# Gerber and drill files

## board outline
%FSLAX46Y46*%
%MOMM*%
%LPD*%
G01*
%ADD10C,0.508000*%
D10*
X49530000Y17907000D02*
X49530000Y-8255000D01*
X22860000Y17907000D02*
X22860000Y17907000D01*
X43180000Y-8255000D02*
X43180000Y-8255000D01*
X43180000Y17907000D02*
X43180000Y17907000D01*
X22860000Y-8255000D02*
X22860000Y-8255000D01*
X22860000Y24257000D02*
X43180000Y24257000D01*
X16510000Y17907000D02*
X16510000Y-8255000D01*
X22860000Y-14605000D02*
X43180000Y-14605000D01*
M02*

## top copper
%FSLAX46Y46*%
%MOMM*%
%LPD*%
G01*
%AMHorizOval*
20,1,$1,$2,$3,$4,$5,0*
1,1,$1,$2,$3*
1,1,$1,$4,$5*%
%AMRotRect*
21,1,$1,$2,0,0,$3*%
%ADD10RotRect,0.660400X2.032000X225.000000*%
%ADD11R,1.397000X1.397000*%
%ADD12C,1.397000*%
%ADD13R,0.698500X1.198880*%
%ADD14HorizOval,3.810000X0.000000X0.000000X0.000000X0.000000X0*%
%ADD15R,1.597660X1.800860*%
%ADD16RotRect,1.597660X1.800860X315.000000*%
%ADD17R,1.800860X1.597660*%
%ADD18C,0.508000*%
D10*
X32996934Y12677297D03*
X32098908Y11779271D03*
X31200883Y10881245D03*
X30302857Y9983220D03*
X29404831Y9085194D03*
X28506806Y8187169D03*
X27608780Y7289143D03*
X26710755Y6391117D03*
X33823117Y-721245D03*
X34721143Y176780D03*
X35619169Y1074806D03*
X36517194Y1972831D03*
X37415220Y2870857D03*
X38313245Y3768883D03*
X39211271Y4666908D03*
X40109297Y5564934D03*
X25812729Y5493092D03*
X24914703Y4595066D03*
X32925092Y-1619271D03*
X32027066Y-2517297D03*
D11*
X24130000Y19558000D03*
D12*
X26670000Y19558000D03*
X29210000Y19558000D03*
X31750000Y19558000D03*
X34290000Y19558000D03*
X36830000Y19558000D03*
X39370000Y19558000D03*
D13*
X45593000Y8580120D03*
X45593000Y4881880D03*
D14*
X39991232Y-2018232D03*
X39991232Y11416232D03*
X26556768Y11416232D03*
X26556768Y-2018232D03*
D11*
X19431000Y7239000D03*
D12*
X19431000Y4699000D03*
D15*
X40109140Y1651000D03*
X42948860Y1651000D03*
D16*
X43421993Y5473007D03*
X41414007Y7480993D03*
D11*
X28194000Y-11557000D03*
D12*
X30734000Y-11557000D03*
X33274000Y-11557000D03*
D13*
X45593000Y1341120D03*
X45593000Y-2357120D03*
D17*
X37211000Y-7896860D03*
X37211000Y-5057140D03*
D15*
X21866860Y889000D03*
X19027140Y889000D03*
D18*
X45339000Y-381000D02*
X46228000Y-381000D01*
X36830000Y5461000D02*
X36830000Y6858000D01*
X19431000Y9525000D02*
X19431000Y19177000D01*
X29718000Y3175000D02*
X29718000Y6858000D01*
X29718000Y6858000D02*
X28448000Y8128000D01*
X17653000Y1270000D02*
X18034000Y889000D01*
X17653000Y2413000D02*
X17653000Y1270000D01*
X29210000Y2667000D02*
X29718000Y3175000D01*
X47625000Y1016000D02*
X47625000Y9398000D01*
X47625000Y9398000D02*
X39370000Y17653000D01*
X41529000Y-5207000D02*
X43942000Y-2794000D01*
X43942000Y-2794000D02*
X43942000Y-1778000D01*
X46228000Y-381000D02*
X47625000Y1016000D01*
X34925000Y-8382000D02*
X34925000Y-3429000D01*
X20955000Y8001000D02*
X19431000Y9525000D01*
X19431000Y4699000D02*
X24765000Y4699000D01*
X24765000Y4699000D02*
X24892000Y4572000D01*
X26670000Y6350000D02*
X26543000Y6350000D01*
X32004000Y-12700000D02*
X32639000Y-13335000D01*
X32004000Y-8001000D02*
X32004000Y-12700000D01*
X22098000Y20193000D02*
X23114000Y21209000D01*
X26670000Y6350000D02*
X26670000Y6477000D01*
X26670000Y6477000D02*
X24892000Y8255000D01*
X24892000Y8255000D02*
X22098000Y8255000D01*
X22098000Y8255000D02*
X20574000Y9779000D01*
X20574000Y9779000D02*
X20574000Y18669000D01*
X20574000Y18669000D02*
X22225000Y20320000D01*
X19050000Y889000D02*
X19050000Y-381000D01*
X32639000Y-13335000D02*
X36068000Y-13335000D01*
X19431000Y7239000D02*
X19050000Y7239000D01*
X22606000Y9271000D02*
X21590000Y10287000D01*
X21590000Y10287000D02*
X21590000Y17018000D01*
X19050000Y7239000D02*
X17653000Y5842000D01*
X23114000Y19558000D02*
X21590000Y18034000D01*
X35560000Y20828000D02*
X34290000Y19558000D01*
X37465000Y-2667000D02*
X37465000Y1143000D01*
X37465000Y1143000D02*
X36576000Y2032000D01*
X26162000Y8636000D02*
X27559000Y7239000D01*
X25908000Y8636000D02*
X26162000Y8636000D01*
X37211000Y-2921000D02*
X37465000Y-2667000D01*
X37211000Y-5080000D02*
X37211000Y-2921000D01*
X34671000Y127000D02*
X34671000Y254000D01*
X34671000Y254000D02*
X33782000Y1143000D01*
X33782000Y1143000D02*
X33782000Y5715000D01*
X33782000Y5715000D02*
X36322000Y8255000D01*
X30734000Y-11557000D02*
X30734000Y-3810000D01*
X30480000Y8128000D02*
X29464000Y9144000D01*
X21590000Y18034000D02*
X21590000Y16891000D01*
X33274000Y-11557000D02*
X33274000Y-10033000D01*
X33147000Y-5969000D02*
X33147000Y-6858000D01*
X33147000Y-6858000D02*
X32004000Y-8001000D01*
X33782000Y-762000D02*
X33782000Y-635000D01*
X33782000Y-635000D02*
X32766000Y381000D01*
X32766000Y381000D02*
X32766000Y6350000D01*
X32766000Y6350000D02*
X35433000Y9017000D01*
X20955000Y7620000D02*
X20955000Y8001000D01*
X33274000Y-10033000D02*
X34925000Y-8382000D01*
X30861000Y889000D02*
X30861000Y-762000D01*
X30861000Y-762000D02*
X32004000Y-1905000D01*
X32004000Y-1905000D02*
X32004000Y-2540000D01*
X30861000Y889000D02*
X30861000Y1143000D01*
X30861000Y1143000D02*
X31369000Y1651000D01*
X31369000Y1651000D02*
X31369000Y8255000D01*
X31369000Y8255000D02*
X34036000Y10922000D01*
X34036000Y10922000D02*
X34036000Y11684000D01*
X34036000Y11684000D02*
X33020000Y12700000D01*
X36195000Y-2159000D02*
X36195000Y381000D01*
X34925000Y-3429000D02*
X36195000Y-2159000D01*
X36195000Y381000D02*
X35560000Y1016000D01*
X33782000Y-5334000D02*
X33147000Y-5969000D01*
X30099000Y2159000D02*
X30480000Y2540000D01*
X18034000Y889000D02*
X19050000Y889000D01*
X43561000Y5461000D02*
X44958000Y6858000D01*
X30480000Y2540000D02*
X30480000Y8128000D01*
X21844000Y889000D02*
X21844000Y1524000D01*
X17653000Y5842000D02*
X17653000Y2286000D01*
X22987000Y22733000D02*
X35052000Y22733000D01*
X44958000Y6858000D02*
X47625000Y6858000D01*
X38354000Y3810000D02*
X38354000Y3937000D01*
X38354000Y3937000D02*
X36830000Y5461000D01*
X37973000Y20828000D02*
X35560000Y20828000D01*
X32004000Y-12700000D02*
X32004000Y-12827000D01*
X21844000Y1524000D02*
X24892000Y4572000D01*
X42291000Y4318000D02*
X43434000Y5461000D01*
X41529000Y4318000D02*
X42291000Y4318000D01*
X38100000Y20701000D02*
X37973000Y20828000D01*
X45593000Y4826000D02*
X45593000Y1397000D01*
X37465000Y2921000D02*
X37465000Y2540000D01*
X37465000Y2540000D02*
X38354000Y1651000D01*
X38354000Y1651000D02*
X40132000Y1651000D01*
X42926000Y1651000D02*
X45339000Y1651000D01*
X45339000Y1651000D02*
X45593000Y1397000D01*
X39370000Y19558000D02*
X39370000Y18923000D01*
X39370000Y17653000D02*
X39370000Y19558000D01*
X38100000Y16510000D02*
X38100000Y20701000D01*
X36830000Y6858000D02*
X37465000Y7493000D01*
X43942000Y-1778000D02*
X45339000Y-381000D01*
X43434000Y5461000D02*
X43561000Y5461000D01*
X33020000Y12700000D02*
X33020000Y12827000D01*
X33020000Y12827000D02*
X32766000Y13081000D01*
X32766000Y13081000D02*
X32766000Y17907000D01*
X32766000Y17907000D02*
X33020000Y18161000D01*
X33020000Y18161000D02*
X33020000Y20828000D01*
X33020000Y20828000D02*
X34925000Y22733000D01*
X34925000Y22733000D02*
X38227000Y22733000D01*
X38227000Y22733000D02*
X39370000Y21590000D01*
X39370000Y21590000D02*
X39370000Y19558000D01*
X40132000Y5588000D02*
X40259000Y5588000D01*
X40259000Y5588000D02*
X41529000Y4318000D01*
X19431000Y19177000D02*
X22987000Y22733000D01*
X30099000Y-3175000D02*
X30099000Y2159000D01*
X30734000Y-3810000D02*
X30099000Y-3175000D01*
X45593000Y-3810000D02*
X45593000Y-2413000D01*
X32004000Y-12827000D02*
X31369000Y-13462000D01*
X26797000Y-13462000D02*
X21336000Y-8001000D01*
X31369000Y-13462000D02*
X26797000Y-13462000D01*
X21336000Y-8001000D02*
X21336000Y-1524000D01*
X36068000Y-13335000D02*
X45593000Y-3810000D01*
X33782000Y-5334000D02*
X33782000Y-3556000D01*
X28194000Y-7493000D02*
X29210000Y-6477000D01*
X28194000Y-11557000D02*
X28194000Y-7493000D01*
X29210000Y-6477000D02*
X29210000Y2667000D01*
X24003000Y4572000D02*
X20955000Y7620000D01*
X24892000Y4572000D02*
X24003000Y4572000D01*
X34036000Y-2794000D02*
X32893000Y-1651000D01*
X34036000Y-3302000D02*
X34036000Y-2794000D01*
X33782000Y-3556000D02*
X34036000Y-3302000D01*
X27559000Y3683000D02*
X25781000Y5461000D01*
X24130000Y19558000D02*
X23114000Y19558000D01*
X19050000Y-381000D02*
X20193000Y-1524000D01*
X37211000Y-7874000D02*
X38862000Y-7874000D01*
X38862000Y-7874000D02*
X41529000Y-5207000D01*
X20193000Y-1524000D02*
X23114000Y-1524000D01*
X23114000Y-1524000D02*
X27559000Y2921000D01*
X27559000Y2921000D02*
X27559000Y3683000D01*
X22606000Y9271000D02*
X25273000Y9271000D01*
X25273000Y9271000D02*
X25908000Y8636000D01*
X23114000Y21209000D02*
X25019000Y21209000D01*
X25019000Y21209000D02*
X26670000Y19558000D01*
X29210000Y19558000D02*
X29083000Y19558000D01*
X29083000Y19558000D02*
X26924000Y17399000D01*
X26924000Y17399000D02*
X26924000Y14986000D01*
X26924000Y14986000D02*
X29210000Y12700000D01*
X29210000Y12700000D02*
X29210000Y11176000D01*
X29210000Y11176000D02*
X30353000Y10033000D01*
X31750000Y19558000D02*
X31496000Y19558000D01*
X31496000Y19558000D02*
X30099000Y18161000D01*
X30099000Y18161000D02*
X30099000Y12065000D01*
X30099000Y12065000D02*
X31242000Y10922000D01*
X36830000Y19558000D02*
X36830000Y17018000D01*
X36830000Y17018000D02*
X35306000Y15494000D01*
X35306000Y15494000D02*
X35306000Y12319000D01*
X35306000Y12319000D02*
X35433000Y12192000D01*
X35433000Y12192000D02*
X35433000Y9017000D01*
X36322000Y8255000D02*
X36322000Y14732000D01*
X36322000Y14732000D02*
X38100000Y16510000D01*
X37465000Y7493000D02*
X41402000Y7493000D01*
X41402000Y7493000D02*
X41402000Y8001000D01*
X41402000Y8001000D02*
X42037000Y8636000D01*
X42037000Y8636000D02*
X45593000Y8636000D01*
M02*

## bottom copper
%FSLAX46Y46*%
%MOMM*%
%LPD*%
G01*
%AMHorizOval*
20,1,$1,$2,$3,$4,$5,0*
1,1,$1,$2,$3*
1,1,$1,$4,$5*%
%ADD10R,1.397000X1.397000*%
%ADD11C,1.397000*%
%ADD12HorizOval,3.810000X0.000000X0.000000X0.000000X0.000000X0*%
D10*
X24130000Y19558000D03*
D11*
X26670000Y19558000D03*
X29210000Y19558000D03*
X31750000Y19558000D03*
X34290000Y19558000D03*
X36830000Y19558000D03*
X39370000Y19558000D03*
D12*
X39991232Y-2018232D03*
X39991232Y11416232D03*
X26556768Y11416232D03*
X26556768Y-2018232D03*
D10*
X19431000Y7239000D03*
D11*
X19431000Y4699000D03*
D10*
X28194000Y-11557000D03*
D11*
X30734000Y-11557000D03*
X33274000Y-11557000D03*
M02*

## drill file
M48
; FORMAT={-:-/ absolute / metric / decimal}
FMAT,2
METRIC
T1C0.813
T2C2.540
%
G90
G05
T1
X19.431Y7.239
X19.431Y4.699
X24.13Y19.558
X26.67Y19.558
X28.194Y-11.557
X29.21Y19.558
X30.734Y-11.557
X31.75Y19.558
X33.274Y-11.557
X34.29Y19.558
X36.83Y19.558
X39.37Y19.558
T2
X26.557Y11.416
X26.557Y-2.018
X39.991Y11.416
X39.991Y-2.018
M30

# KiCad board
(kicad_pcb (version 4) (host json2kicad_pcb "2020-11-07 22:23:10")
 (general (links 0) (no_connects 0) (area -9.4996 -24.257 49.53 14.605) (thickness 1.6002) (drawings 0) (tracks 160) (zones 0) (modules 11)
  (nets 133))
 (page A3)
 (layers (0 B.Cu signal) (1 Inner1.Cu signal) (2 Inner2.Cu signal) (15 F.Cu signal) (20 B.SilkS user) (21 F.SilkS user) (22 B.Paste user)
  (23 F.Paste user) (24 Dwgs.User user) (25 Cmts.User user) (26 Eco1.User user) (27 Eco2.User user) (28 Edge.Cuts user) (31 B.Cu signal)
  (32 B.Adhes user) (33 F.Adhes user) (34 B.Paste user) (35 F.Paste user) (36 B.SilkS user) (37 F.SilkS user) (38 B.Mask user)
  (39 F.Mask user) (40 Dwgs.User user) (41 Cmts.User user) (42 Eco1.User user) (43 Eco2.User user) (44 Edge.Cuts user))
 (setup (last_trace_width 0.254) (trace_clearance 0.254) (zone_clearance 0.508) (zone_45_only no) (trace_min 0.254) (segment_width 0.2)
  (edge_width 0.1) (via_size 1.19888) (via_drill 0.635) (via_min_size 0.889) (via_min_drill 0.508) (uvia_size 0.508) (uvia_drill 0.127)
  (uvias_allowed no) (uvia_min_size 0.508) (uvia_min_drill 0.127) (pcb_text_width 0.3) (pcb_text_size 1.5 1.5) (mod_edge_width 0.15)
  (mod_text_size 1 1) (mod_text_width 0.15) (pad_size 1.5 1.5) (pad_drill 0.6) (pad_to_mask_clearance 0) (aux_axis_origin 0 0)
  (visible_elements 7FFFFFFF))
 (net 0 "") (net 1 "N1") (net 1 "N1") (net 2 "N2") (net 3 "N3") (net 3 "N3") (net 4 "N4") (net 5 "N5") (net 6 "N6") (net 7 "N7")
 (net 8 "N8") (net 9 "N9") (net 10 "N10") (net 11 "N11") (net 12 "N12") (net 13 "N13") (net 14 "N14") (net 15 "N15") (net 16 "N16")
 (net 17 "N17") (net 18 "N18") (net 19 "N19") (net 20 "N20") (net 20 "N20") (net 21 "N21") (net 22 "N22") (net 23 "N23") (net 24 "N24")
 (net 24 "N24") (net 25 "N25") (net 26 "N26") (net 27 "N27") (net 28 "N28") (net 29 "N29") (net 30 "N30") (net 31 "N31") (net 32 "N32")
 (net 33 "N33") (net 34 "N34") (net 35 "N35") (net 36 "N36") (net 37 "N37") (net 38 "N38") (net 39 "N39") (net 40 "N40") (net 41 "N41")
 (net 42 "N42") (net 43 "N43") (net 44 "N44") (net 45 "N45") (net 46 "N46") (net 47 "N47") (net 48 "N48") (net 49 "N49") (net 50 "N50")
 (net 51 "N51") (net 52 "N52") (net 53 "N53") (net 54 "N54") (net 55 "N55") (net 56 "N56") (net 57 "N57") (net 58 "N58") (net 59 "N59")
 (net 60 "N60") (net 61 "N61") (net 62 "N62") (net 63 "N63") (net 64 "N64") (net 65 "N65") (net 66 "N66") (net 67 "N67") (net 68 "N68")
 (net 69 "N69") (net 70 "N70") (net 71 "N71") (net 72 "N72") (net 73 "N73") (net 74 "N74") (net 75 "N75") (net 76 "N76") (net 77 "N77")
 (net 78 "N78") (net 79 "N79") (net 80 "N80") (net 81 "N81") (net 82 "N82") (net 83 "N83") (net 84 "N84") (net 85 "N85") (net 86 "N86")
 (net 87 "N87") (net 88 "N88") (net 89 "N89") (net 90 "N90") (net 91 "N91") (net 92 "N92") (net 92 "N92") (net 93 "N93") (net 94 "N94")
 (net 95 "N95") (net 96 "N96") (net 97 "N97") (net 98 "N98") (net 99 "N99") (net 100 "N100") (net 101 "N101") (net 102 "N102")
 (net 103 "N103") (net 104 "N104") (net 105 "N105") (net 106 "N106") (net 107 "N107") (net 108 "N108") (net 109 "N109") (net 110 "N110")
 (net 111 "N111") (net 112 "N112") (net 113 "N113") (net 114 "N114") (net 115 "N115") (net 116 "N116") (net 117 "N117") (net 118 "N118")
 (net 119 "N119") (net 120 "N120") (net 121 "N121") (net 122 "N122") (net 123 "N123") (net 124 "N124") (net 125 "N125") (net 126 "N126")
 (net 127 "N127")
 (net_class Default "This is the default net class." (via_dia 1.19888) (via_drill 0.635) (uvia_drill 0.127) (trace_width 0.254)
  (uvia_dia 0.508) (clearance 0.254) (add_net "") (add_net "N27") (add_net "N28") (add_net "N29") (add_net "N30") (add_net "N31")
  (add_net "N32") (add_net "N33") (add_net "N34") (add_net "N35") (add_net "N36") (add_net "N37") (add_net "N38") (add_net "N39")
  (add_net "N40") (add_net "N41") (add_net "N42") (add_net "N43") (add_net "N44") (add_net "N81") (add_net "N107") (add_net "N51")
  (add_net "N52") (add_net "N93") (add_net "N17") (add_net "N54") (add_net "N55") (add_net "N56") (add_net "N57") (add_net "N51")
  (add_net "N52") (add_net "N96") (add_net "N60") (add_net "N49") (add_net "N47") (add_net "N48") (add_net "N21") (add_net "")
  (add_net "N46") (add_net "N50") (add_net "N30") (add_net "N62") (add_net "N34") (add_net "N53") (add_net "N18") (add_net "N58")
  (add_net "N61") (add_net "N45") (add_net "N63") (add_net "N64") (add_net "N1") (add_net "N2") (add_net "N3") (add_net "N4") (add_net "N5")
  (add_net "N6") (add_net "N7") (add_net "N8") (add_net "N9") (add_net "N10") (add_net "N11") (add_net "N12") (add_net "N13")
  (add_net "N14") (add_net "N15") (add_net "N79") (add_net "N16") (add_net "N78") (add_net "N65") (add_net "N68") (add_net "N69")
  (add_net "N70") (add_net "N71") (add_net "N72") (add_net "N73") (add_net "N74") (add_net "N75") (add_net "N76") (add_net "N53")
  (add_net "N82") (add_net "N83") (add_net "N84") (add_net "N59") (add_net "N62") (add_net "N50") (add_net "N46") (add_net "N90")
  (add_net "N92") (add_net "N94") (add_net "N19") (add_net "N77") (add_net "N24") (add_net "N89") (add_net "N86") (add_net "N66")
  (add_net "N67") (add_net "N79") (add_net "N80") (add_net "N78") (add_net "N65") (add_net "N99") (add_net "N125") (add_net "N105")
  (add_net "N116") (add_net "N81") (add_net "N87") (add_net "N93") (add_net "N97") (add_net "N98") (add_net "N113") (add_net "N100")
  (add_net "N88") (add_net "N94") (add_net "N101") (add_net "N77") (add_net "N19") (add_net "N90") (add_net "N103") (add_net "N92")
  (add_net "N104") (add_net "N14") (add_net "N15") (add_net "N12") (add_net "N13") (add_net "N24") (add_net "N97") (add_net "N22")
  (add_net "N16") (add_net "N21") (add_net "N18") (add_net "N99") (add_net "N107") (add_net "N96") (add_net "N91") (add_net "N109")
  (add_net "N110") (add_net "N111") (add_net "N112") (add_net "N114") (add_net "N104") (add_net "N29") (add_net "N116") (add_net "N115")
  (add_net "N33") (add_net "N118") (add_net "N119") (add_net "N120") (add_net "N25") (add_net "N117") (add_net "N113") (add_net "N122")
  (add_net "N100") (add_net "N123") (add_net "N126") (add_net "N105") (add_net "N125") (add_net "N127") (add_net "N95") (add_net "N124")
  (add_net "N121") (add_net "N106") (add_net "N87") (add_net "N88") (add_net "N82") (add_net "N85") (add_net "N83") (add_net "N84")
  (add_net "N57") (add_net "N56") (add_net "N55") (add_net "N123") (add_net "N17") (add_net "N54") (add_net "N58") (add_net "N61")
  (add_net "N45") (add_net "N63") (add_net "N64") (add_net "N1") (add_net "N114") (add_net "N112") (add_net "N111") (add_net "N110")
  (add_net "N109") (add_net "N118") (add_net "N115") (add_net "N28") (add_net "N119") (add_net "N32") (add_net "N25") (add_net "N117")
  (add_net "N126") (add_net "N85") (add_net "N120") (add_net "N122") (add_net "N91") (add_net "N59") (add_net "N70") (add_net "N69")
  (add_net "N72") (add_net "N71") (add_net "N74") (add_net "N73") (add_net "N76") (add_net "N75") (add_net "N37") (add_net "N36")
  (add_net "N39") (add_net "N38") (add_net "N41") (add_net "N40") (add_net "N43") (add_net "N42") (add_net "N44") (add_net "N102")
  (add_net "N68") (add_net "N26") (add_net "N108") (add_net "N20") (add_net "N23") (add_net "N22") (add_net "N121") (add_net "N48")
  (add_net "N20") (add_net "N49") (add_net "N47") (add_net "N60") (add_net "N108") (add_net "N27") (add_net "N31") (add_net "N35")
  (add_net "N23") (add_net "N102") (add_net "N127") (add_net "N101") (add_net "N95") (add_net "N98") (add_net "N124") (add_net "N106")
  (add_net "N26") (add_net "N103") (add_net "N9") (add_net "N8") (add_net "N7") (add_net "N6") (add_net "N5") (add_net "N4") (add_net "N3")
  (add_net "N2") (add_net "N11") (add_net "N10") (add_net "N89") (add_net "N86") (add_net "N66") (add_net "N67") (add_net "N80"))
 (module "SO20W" (layer "F.Cu") (at 32.512 -5.08 -135.00)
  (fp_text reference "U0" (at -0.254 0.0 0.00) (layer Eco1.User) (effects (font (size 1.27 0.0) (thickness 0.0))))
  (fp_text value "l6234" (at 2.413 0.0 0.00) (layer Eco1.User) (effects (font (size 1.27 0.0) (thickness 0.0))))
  (pad 1 smd rect (at -5.715 5.0292 -135.00) (size 0.6604 2.032) (drill 0.0) (layers "F.Cu" "F.Paste") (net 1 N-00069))
  (pad 2 smd rect (at -4.445 5.0292 -135.00) (size 0.6604 2.032) (drill 0.0) (layers "F.Cu" "F.Paste") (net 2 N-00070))
  (pad 3 smd rect (at -3.175 5.0292 -135.00) (size 0.6604 2.032) (drill 0.0) (layers "F.Cu" "F.Paste") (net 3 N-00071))
  (pad 4 smd rect (at -1.905 5.0292 -135.00) (size 0.6604 2.032) (drill 0.0) (layers "F.Cu" "F.Paste") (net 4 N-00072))
  (pad 5 smd rect (at -0.635 5.0292 -135.00) (size 0.6604 2.032) (drill 0.0) (layers "F.Cu" "F.Paste") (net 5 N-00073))
  (pad 6 smd rect (at 0.635 5.0292 -135.00) (size 0.6604 2.032) (drill 0.0) (layers "F.Cu" "F.Paste") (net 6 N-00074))
  (pad 7 smd rect (at 1.905 5.0292 -135.00) (size 0.6604 2.032) (drill 0.0) (layers "F.Cu" "F.Paste") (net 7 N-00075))
  (pad 8 smd rect (at 3.175 5.0292 -135.00) (size 0.6604 2.032) (drill 0.0) (layers "F.Cu" "F.Paste") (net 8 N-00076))
  (pad 13 smd rect (at 3.175 -5.0292 -135.00) (size 0.6604 2.032) (drill 0.0) (layers "F.Cu" "F.Paste") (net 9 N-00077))
  (pad 14 smd rect (at 1.905 -5.0292 -135.00) (size 0.6604 2.032) (drill 0.0) (layers "F.Cu" "F.Paste") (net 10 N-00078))
  (pad 15 smd rect (at 0.635 -5.0292 -135.00) (size 0.6604 2.032) (drill 0.0) (layers "F.Cu" "F.Paste") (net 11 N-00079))
  (pad 16 smd rect (at -0.635 -5.0292 -135.00) (size 0.6604 2.032) (drill 0.0) (layers "F.Cu" "F.Paste") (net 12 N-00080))
  (pad 17 smd rect (at -1.905 -5.0292 -135.00) (size 0.6604 2.032) (drill 0.0) (layers "F.Cu" "F.Paste") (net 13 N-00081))
  (pad 18 smd rect (at -3.175 -5.0292 -135.00) (size 0.6604 2.032) (drill 0.0) (layers "F.Cu" "F.Paste") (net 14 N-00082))
  (pad 19 smd rect (at -4.445 -5.0292 -135.00) (size 0.6604 2.032) (drill 0.0) (layers "F.Cu" "F.Paste") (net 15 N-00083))
  (pad 20 smd rect (at -5.715 -5.0292 -135.00) (size 0.6604 2.032) (drill 0.0) (layers "F.Cu" "F.Paste") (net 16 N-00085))
  (pad 9 smd rect (at 4.445 5.0292 -135.00) (size 0.6604 2.032) (drill 0.0) (layers "F.Cu" "F.Paste") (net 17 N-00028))
  (pad 10 smd rect (at 5.715 5.0292 -135.00) (size 0.6604 2.032) (drill 0.0) (layers "F.Cu" "F.Paste") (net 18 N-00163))
  (pad 12 smd rect (at 4.445 -5.0292 -135.00) (size 0.6604 2.032) (drill 0.0) (layers "F.Cu" "F.Paste") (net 17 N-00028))
  (pad 11 smd rect (at 5.715 -5.0292 -135.00) (size 0.6604 2.032) (drill 0.0) (layers "F.Cu" "F.Paste") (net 1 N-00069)))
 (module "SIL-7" (layer "F.Cu") (at 31.75 -19.558 0.00)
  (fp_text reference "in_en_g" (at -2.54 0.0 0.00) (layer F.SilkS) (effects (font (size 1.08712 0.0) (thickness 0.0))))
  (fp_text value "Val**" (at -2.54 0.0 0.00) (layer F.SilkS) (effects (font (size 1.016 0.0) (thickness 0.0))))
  (pad 1 thru_hole rect (at -7.62 0.0 0.00) (size 1.397 1.397) (drill 0.8128)
   (layers "B.Cu" "Inner1.Cu" "Inner2.Cu" "F.Cu" "F.SilkS" "B.Paste" "F.Paste") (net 7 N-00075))
  (pad 2 thru_hole circle (at -5.08 0.0 0.00) (size 1.397 1.397) (drill 0.8128)
   (layers "B.Cu" "Inner1.Cu" "Inner2.Cu" "F.Cu" "B.SilkS" "F.SilkS" "B.Paste" "F.Paste") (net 8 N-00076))
  (pad 3 thru_hole circle (at -2.54 0.0 0.00) (size 1.397 1.397) (drill 0.8128)
   (layers "B.Cu" "Inner1.Cu" "Inner2.Cu" "F.Cu" "B.SilkS" "F.SilkS" "B.Paste" "F.Paste") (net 4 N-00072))
  (pad 4 thru_hole circle (at 0.0 0.0 0.00) (size 1.397 1.397) (drill 0.8128)
   (layers "B.Cu" "Inner1.Cu" "Inner2.Cu" "F.Cu" "B.SilkS" "F.SilkS" "B.Paste" "F.Paste") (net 3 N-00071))
  (pad 5 thru_hole circle (at 2.54 0.0 0.00) (size 1.397 1.397) (drill 0.8128)
   (layers "B.Cu" "Inner1.Cu" "Inner2.Cu" "F.Cu" "B.SilkS" "F.SilkS" "B.Paste" "F.Paste") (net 10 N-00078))
  (pad 6 thru_hole circle (at 5.08 0.0 0.00) (size 1.397 1.397) (drill 0.8128)
   (layers "B.Cu" "Inner1.Cu" "Inner2.Cu" "F.Cu" "B.SilkS" "F.SilkS" "B.Paste" "F.Paste") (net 9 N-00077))
  (pad 7 thru_hole circle (at 7.62 0.0 0.00) (size 1.397 1.397) (drill 0.8128)
   (layers "B.Cu" "Inner1.Cu" "Inner2.Cu" "F.Cu" "B.SilkS" "F.SilkS" "B.Paste" "F.Paste") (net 1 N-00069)))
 (segment (start 45.339 0.381) (end 46.228 0.381) (width 0.508) (layer F.Cu) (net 1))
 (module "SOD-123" (layer "F.Cu") (at 45.593 -6.731 -90.00)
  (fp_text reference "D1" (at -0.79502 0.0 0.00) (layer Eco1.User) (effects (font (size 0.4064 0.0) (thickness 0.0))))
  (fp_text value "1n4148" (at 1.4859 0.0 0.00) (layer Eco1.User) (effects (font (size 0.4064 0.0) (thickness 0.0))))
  (pad C smd rect (at -1.84912 0.0 -90.00) (size 1.19888 0.6985) (drill 0.0) (layers "F.Cu" "F.Paste") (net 14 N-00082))
  (pad A smd rect (at 1.84912 0.0 -90.00) (size 1.19888 0.6985) (drill 0.0) (layers "F.Cu" "F.Paste") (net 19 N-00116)))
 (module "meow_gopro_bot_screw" (layer "F.Cu") (at 33.274 -4.699 45.00)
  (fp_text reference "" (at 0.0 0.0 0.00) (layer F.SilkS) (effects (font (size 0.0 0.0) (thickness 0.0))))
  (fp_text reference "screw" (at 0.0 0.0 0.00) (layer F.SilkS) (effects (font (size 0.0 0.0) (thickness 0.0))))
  (pad S0 thru_hole oval (at 0.0 9.4996 45.00) (size 3.81 3.81) (drill 2.54)
   (layers "B.Cu" "Inner1.Cu" "Inner2.Cu" "F.Cu" "B.Paste" "F.Paste") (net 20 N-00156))
  (pad S1 thru_hole oval (at 9.4996 0.0 45.00) (size 3.81 3.81) (drill 2.54)
   (layers "B.Cu" "Inner1.Cu" "Inner2.Cu" "F.Cu" "B.Paste" "F.Paste") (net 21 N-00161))
  (pad S2 thru_hole oval (at 0.0 -9.4996 45.00) (size 3.81 3.81) (drill 2.54)
   (layers "B.Cu" "Inner1.Cu" "Inner2.Cu" "F.Cu" "B.Paste" "F.Paste") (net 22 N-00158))
  (pad S3 thru_hole oval (at -9.4996 0.0 45.00) (size 3.81 3.81) (drill 2.54)
   (layers "B.Cu" "Inner1.Cu" "Inner2.Cu" "F.Cu" "B.Paste" "F.Paste") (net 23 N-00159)))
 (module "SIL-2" (layer "F.Cu") (at 19.431 -5.969 -90.00)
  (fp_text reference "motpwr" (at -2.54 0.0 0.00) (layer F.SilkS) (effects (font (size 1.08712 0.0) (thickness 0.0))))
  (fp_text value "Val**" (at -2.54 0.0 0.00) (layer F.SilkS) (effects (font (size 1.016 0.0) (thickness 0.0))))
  (pad 1 thru_hole rect (at -1.27 0.0 -90.00) (size 1.397 1.397) (drill 0.8128)
   (layers "B.Cu" "Inner1.Cu" "Inner2.Cu" "F.Cu" "F.SilkS" "B.Paste" "F.Paste") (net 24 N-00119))
  (pad 2 thru_hole circle (at 1.27 0.0 -90.00) (size 1.397 1.397) (drill 0.8128)
   (layers "B.Cu" "Inner1.Cu" "Inner2.Cu" "F.Cu" "F.SilkS" "B.Paste" "F.Paste") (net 18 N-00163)))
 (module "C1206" (layer "F.Cu") (at 41.529 -1.651 180.00)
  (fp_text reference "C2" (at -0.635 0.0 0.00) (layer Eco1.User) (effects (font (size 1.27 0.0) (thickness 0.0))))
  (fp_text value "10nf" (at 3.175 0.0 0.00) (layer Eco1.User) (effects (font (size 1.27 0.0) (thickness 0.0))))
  (pad 2 smd rect (at 1.41986 0.0 -180.00) (size 1.59766 1.80086) (drill 0.0) (layers "F.Cu" "F.Paste") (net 13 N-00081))
  (pad 1 smd rect (at -1.41986 0.0 -180.00) (size 1.59766 1.80086) (drill 0.0) (layers "F.Cu" "F.Paste") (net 19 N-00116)))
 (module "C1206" (layer "F.Cu") (at 42.418 -6.477 -45.00)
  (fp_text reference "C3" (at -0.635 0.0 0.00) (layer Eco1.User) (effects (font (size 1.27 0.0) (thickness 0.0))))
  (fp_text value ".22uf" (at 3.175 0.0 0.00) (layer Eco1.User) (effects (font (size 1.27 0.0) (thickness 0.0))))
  (pad 2 smd rect (at 1.41986 0.0 -45.00) (size 1.59766 1.80086) (drill 0.0) (layers "F.Cu" "F.Paste") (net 16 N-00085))
  (pad 1 smd rect (at -1.41986 0.0 -45.00) (size 1.59766 1.80086) (drill 0.0) (layers "F.Cu" "F.Paste") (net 14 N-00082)))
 (segment (start 36.83 -5.461) (end 36.83 -6.858) (width 0.508) (layer F.Cu) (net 14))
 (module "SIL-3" (layer "F.Cu") (at 30.734 11.557 0.00)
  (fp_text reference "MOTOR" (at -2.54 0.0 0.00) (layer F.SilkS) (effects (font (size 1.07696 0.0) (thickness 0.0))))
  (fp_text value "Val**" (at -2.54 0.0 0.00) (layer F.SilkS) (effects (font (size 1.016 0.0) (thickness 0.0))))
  (pad 1 thru_hole rect (at -2.54 0.0 0.00) (size 1.397 1.397) (drill 0.8128)
   (layers "B.Cu" "Inner1.Cu" "Inner2.Cu" "F.Cu" "F.SilkS" "B.Paste" "F.Paste") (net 6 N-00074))
  (pad 2 thru_hole circle (at 0.0 0.0 0.00) (size 1.397 1.397) (drill 0.8128)
   (layers "B.Cu" "Inner1.Cu" "Inner2.Cu" "F.Cu" "F.SilkS" "B.Paste" "F.Paste") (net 5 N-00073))
  (pad 3 thru_hole circle (at 2.54 0.0 0.00) (size 1.397 1.397) (drill 0.8128)
   (layers "B.Cu" "Inner1.Cu" "Inner2.Cu" "F.Cu" "F.SilkS" "B.Paste" "F.Paste") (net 11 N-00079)))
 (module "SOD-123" (layer "F.Cu") (at 45.593 0.508 -90.00)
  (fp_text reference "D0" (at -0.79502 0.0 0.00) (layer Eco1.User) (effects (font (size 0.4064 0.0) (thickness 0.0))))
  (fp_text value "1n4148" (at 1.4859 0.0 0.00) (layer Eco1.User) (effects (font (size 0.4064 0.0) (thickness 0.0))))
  (pad C smd rect (at -1.84912 0.0 -90.00) (size 1.19888 0.6985) (drill 0.0) (layers "F.Cu" "F.Paste") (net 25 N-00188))
  (pad A smd rect (at 1.84912 0.0 -90.00) (size 1.19888 0.6985) (drill 0.0) (layers "F.Cu" "F.Paste") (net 17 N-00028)))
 (gr_line (start 49.53 -17.907) (end 49.53 8.255) (angle 51566.20) (width 0.508) (layer Edge.Cuts))
 (gr_line (start 22.86 -17.907) (end 22.86 -17.907) (angle -90.00) (width 0.508) (layer Edge.Cuts))
 (gr_line (start 43.18 8.255) (end 43.18 8.255) (angle -90.00) (width 0.508) (layer Edge.Cuts))
 (gr_line (start 43.18 -17.907) (end 43.18 -17.907) (angle -90.00) (width 0.508) (layer Edge.Cuts))
 (gr_line (start 22.86 8.255) (end 22.86 8.255) (angle -90.00) (width 0.508) (layer Edge.Cuts))
 (segment (start 19.431 -9.525) (end 19.431 -19.177) (width 0.508) (layer F.Cu) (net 1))
 (segment (start 29.718 -3.175) (end 29.718 -6.858) (width 0.508) (layer F.Cu) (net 6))
 (segment (start 29.718 -6.858) (end 28.448 -8.128) (width 0.508) (layer F.Cu) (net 6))
 (segment (start 17.653 -1.27) (end 18.034 -0.889) (width 0.508) (layer F.Cu) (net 17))
 (segment (start 17.653 -2.413) (end 17.653 -1.27) (width 0.508) (layer F.Cu) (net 17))
 (segment (start 29.21 -2.667) (end 29.718 -3.175) (width 0.508) (layer F.Cu) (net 6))
 (segment (start 47.625 -1.016) (end 47.625 -9.398) (width 0.508) (layer F.Cu) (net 1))
 (segment (start 47.625 -9.398) (end 39.37 -17.653) (width 0.508) (layer F.Cu) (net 1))
 (segment (start 41.529 5.207) (end 43.942 2.794) (width 0.508) (layer F.Cu) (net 1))
 (segment (start 43.942 2.794) (end 43.942 1.778) (width 0.508) (layer F.Cu) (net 1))
 (segment (start 46.228 0.381) (end 47.625 -1.016) (width 0.508) (layer F.Cu) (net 1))
 (segment (start 34.925 8.382) (end 34.925 3.429) (width 0.508) (layer F.Cu) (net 11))
 (segment (start 20.955 -8.001) (end 19.431 -9.525) (width 0.508) (layer F.Cu) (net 1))
 (segment (start 19.431 -4.699) (end 24.765 -4.699) (width 0.508) (layer F.Cu) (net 18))
 (segment (start 24.765 -4.699) (end 24.892 -4.572) (width 0.508) (layer F.Cu) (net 18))
 (segment (start 26.67 -6.35) (end 26.543 -6.35) (width 0.508) (layer F.Cu) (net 8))
 (segment (start 32.004 12.7) (end 32.639 13.335) (width 0.508) (layer F.Cu) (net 17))
 (segment (start 32.004 8.001) (end 32.004 12.7) (width 0.508) (layer F.Cu) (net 17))
 (segment (start 22.098 -20.193) (end 23.114 -21.209) (width 0.508) (layer F.Cu) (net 8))
 (segment (start 26.67 -6.35) (end 26.67 -6.477) (width 0.508) (layer F.Cu) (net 8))
 (segment (start 26.67 -6.477) (end 24.892 -8.255) (width 0.508) (layer F.Cu) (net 8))
 (segment (start 24.892 -8.255) (end 22.098 -8.255) (width 0.508) (layer F.Cu) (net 8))
 (segment (start 22.098 -8.255) (end 20.574 -9.779) (width 0.508) (layer F.Cu) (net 8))
 (segment (start 20.574 -9.779) (end 20.574 -18.669) (width 0.508) (layer F.Cu) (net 8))
 (segment (start 20.574 -18.669) (end 22.225 -20.32) (width 0.508) (layer F.Cu) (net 8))
 (segment (start 19.05 -0.889) (end 19.05 0.381) (width 0.508) (layer F.Cu) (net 17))
 (segment (start 32.639 13.335) (end 36.068 13.335) (width 0.508) (layer F.Cu) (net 17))
 (segment (start 19.431 -7.239) (end 19.05 -7.239) (width 0.508) (layer F.Cu) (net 17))
 (segment (start 22.606 -9.271) (end 21.59 -10.287) (width 0.508) (layer F.Cu) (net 7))
 (segment (start 21.59 -10.287) (end 21.59 -17.018) (width 0.508) (layer F.Cu) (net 7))
 (segment (start 19.05 -7.239) (end 17.653 -5.842) (width 0.508) (layer F.Cu) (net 17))
 (segment (start 23.114 -19.558) (end 21.59 -18.034) (width 0.508) (layer F.Cu) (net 7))
 (segment (start 35.56 -20.828) (end 34.29 -19.558) (width 0.508) (layer F.Cu) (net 10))
 (segment (start 37.465 2.667) (end 37.465 -1.143) (width 0.508) (layer F.Cu) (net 12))
 (segment (start 37.465 -1.143) (end 36.576 -2.032) (width 0.508) (layer F.Cu) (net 12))
 (segment (start 26.162 -8.636) (end 27.559 -7.239) (width 0.508) (layer F.Cu) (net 7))
 (segment (start 25.908 -8.636) (end 26.162 -8.636) (width 0.508) (layer F.Cu) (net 7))
 (segment (start 37.211 2.921) (end 37.465 2.667) (width 0.508) (layer F.Cu) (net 12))
 (segment (start 37.211 5.08) (end 37.211 2.921) (width 0.508) (layer F.Cu) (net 12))
 (segment (start 34.671 -0.127) (end 34.671 -0.254) (width 0.508) (layer F.Cu) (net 10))
 (segment (start 34.671 -0.254) (end 33.782 -1.143) (width 0.508) (layer F.Cu) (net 10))
 (segment (start 33.782 -1.143) (end 33.782 -5.715) (width 0.508) (layer F.Cu) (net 10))
 (segment (start 33.782 -5.715) (end 36.322 -8.255) (width 0.508) (layer F.Cu) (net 10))
 (segment (start 30.734 11.557) (end 30.734 3.81) (width 0.508) (layer F.Cu) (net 5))
 (segment (start 30.48 -8.128) (end 29.464 -9.144) (width 0.508) (layer F.Cu) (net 5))
 (segment (start 21.59 -18.034) (end 21.59 -16.891) (width 0.508) (layer F.Cu) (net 7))
 (segment (start 33.274 11.557) (end 33.274 10.033) (width 0.508) (layer F.Cu) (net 11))
 (segment (start 33.147 5.969) (end 33.147 6.858) (width 0.508) (layer F.Cu) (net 17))
 (segment (start 33.147 6.858) (end 32.004 8.001) (width 0.508) (layer F.Cu) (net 17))
 (segment (start 33.782 0.762) (end 33.782 0.635) (width 0.508) (layer F.Cu) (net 9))
 (segment (start 33.782 0.635) (end 32.766 -0.381) (width 0.508) (layer F.Cu) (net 9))
 (segment (start 32.766 -0.381) (end 32.766 -6.35) (width 0.508) (layer F.Cu) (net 9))
 (segment (start 32.766 -6.35) (end 35.433 -9.017) (width 0.508) (layer F.Cu) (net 9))
 (segment (start 20.955 -7.62) (end 20.955 -8.001) (width 0.508) (layer F.Cu) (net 1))
 (segment (start 33.274 10.033) (end 34.925 8.382) (width 0.508) (layer F.Cu) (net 11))
 (segment (start 30.861 -0.889) (end 30.861 0.762) (width 0.508) (layer F.Cu) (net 1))
 (segment (start 30.861 0.762) (end 32.004 1.905) (width 0.508) (layer F.Cu) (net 1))
 (segment (start 32.004 1.905) (end 32.004 2.54) (width 0.508) (layer F.Cu) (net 1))
 (segment (start 30.861 -0.889) (end 30.861 -1.143) (width 0.508) (layer F.Cu) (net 1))
 (segment (start 30.861 -1.143) (end 31.369 -1.651) (width 0.508) (layer F.Cu) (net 1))
 (segment (start 31.369 -1.651) (end 31.369 -8.255) (width 0.508) (layer F.Cu) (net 1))
 (segment (start 31.369 -8.255) (end 34.036 -10.922) (width 0.508) (layer F.Cu) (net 1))
 (segment (start 34.036 -10.922) (end 34.036 -11.684) (width 0.508) (layer F.Cu) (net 1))
 (segment (start 34.036 -11.684) (end 33.02 -12.7) (width 0.508) (layer F.Cu) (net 1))
 (segment (start 36.195 2.159) (end 36.195 -0.381) (width 0.508) (layer F.Cu) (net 11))
 (segment (start 34.925 3.429) (end 36.195 2.159) (width 0.508) (layer F.Cu) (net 11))
 (segment (start 36.195 -0.381) (end 35.56 -1.016) (width 0.508) (layer F.Cu) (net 11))
 (segment (start 33.782 5.334) (end 33.147 5.969) (width 0.508) (layer F.Cu) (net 17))
 (segment (start 30.099 -2.159) (end 30.48 -2.54) (width 0.508) (layer F.Cu) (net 5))
 (segment (start 18.034 -0.889) (end 19.05 -0.889) (width 0.508) (layer F.Cu) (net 17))
 (segment (start 43.561 -5.461) (end 44.958 -6.858) (width 0.508) (layer F.Cu) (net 1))
 (segment (start 30.48 -2.54) (end 30.48 -8.128) (width 0.508) (layer F.Cu) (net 5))
 (segment (start 21.844 -0.889) (end 21.844 -1.524) (width 0.508) (layer F.Cu) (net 18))
 (segment (start 17.653 -5.842) (end 17.653 -2.286) (width 0.508) (layer F.Cu) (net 17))
 (segment (start 22.987 -22.733) (end 35.052 -22.733) (width 0.508) (layer F.Cu) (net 1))
 (segment (start 44.958 -6.858) (end 47.625 -6.858) (width 0.508) (layer F.Cu) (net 1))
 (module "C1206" (layer "F.Cu") (at 37.211 6.477 -90.00)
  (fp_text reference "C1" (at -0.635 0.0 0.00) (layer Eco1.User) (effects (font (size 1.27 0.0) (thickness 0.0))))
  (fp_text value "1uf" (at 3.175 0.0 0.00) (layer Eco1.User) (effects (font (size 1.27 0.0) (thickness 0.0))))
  (pad 2 smd rect (at 1.41986 0.0 -90.00) (size 1.59766 1.80086) (drill 0.0) (layers "F.Cu" "F.Paste") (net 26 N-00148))
  (pad 1 smd rect (at -1.41986 0.0 -90.00) (size 1.59766 1.80086) (drill 0.0) (layers "F.Cu" "F.Paste") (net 12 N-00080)))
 (segment (start 38.354 -3.81) (end 38.354 -3.937) (width 0.508) (layer F.Cu) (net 14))
 (segment (start 38.354 -3.937) (end 36.83 -5.461) (width 0.508) (layer F.Cu) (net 14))
 (segment (start 37.973 -20.828) (end 35.56 -20.828) (width 0.508) (layer F.Cu) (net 10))
 (segment (start 32.004 12.7) (end 32.004 12.827) (width 0.508) (layer F.Cu) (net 17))
 (segment (start 21.844 -1.524) (end 24.892 -4.572) (width 0.508) (layer F.Cu) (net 18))
 (segment (start 42.291 -4.318) (end 43.434 -5.461) (width 0.508) (layer F.Cu) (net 16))
 (segment (start 41.529 -4.318) (end 42.291 -4.318) (width 0.508) (layer F.Cu) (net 16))
 (segment (start 38.1 -20.701) (end 37.973 -20.828) (width 0.508) (layer F.Cu) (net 10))
 (segment (start 45.593 -4.826) (end 45.593 -1.397) (width 0.508) (layer F.Cu) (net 19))
 (segment (start 37.465 -2.921) (end 37.465 -2.54) (width 0.508) (layer F.Cu) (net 13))
 (segment (start 37.465 -2.54) (end 38.354 -1.651) (width 0.508) (layer F.Cu) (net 13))
 (segment (start 38.354 -1.651) (end 40.132 -1.651) (width 0.508) (layer F.Cu) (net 13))
 (segment (start 42.926 -1.651) (end 45.339 -1.651) (width 0.508) (layer F.Cu) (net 19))
 (segment (start 45.339 -1.651) (end 45.593 -1.397) (width 0.508) (layer F.Cu) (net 19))
 (segment (start 39.37 -19.558) (end 39.37 -18.923) (width 0.508) (layer F.Cu) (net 1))
 (segment (start 39.37 -17.653) (end 39.37 -19.558) (width 0.508) (layer F.Cu) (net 1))
 (segment (start 38.1 -16.51) (end 38.1 -20.701) (width 0.508) (layer F.Cu) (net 10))
 (segment (start 36.83 -6.858) (end 37.465 -7.493) (width 0.508) (layer F.Cu) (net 14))
 (segment (start 43.942 1.778) (end 45.339 0.381) (width 0.508) (layer F.Cu) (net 1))
 (segment (start 43.434 -5.461) (end 43.561 -5.461) (width 0.508) (layer F.Cu) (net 1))
 (segment (start 33.02 -12.7) (end 33.02 -12.827) (width 0.508) (layer F.Cu) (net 1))
 (segment (start 33.02 -12.827) (end 32.766 -13.081) (width 0.508) (layer F.Cu) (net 1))
 (segment (start 32.766 -13.081) (end 32.766 -17.907) (width 0.508) (layer F.Cu) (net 1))
 (segment (start 32.766 -17.907) (end 33.02 -18.161) (width 0.508) (layer F.Cu) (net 1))
 (segment (start 33.02 -18.161) (end 33.02 -20.828) (width 0.508) (layer F.Cu) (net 1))
 (segment (start 33.02 -20.828) (end 34.925 -22.733) (width 0.508) (layer F.Cu) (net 1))
 (segment (start 34.925 -22.733) (end 38.227 -22.733) (width 0.508) (layer F.Cu) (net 1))
 (segment (start 38.227 -22.733) (end 39.37 -21.59) (width 0.508) (layer F.Cu) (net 1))
 (segment (start 39.37 -21.59) (end 39.37 -19.558) (width 0.508) (layer F.Cu) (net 1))
 (segment (start 40.132 -5.588) (end 40.259 -5.588) (width 0.508) (layer F.Cu) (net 16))
 (segment (start 40.259 -5.588) (end 41.529 -4.318) (width 0.508) (layer F.Cu) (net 16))
 (segment (start 19.431 -19.177) (end 22.987 -22.733) (width 0.508) (layer F.Cu) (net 1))
 (segment (start 30.099 3.175) (end 30.099 -2.159) (width 0.508) (layer F.Cu) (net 5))
 (segment (start 30.734 3.81) (end 30.099 3.175) (width 0.508) (layer F.Cu) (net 5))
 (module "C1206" (layer "F.Cu") (at 20.447 -0.889 0.00)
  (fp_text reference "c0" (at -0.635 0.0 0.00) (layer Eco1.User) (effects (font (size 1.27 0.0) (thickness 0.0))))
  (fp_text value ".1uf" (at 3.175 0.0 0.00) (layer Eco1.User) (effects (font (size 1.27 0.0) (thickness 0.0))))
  (pad 2 smd rect (at 1.41986 0.0 0.00) (size 1.59766 1.80086) (drill 0.0) (layers "F.Cu" "F.Paste") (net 18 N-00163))
  (pad 1 smd rect (at -1.41986 0.0 0.00) (size 1.59766 1.80086) (drill 0.0) (layers "F.Cu" "F.Paste") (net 17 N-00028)))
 (segment (start 45.593 3.81) (end 45.593 2.413) (width 0.508) (layer F.Cu) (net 17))
 (segment (start 32.004 12.827) (end 31.369 13.462) (width 0.508) (layer F.Cu) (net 17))
 (segment (start 26.797 13.462) (end 21.336 8.001) (width 0.508) (layer F.Cu) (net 17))
 (segment (start 31.369 13.462) (end 26.797 13.462) (width 0.508) (layer F.Cu) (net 17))
 (segment (start 21.336 8.001) (end 21.336 1.524) (width 0.508) (layer F.Cu) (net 17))
 (segment (start 36.068 13.335) (end 45.593 3.81) (width 0.508) (layer F.Cu) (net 17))
 (segment (start 33.782 5.334) (end 33.782 3.556) (width 0.508) (layer F.Cu) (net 17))
 (gr_line (start 22.86 -24.257) (end 43.18 -24.257) (angle 51566.20) (width 0.508) (layer Edge.Cuts))
 (segment (start 28.194 7.493) (end 29.21 6.477) (width 0.508) (layer F.Cu) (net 6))
 (segment (start 28.194 11.557) (end 28.194 7.493) (width 0.508) (layer F.Cu) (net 6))
 (segment (start 29.21 6.477) (end 29.21 -2.667) (width 0.508) (layer F.Cu) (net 6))
 (segment (start 24.003 -4.572) (end 20.955 -7.62) (width 0.508) (layer F.Cu) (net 1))
 (segment (start 24.892 -4.572) (end 24.003 -4.572) (width 0.508) (layer F.Cu) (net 1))
 (gr_line (start 16.51 -17.907) (end 16.51 8.255) (angle 51566.20) (width 0.508) (layer Edge.Cuts))
 (gr_line (start 22.86 14.605) (end 43.18 14.605) (angle 51566.20) (width 0.508) (layer Edge.Cuts))
 (segment (start 34.036 2.794) (end 32.893 1.651) (width 0.508) (layer F.Cu) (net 17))
 (segment (start 34.036 3.302) (end 34.036 2.794) (width 0.508) (layer F.Cu) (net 17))
 (segment (start 33.782 3.556) (end 34.036 3.302) (width 0.508) (layer F.Cu) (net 17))
 (segment (start 27.559 -3.683) (end 25.781 -5.461) (width 0.508) (layer F.Cu) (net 17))
 (segment (start 24.13 -19.558) (end 23.114 -19.558) (width 0.508) (layer F.Cu) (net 7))
 (segment (start 19.05 0.381) (end 20.193 1.524) (width 0.508) (layer F.Cu) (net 17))
 (segment (start 37.211 7.874) (end 38.862 7.874) (width 0.508) (layer F.Cu) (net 1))
 (segment (start 38.862 7.874) (end 41.529 5.207) (width 0.508) (layer F.Cu) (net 1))
 (segment (start 20.193 1.524) (end 23.114 1.524) (width 0.508) (layer F.Cu) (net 17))
 (segment (start 23.114 1.524) (end 27.559 -2.921) (width 0.508) (layer F.Cu) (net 17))
 (segment (start 27.559 -2.921) (end 27.559 -3.683) (width 0.508) (layer F.Cu) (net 17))
 (segment (start 22.606 -9.271) (end 25.273 -9.271) (width 0.508) (layer F.Cu) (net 7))
 (segment (start 25.273 -9.271) (end 25.908 -8.636) (width 0.508) (layer F.Cu) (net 7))
 (segment (start 23.114 -21.209) (end 25.019 -21.209) (width 0.508) (layer F.Cu) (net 8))
 (segment (start 25.019 -21.209) (end 26.67 -19.558) (width 0.508) (layer F.Cu) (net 8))
 (segment (start 29.21 -19.558) (end 29.083 -19.558) (width 0.508) (layer F.Cu) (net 4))
 (segment (start 29.083 -19.558) (end 26.924 -17.399) (width 0.508) (layer F.Cu) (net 4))
 (segment (start 26.924 -17.399) (end 26.924 -14.986) (width 0.508) (layer F.Cu) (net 4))
 (segment (start 26.924 -14.986) (end 29.21 -12.7) (width 0.508) (layer F.Cu) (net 4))
 (segment (start 29.21 -12.7) (end 29.21 -11.176) (width 0.508) (layer F.Cu) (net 4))
 (segment (start 29.21 -11.176) (end 30.353 -10.033) (width 0.508) (layer F.Cu) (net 4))
 (segment (start 31.75 -19.558) (end 31.496 -19.558) (width 0.508) (layer F.Cu) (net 3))
 (segment (start 31.496 -19.558) (end 30.099 -18.161) (width 0.508) (layer F.Cu) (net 3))
 (segment (start 30.099 -18.161) (end 30.099 -12.065) (width 0.508) (layer F.Cu) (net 3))
 (segment (start 30.099 -12.065) (end 31.242 -10.922) (width 0.508) (layer F.Cu) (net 3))
 (segment (start 36.83 -19.558) (end 36.83 -17.018) (width 0.508) (layer F.Cu) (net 9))
 (segment (start 36.83 -17.018) (end 35.306 -15.494) (width 0.508) (layer F.Cu) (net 9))
 (segment (start 35.306 -15.494) (end 35.306 -12.319) (width 0.508) (layer F.Cu) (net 9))
 (segment (start 35.306 -12.319) (end 35.433 -12.192) (width 0.508) (layer F.Cu) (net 9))
 (segment (start 35.433 -12.192) (end 35.433 -9.017) (width 0.508) (layer F.Cu) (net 9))
 (segment (start 36.322 -8.255) (end 36.322 -14.732) (width 0.508) (layer F.Cu) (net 10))
 (segment (start 36.322 -14.732) (end 38.1 -16.51) (width 0.508) (layer F.Cu) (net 10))
 (segment (start 37.465 -7.493) (end 41.402 -7.493) (width 0.508) (layer F.Cu) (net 14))
 (segment (start 41.402 -7.493) (end 41.402 -8.001) (width 0.508) (layer F.Cu) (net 14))
 (segment (start 41.402 -8.001) (end 42.037 -8.636) (width 0.508) (layer F.Cu) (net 14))
 (segment (start 42.037 -8.636) (end 45.593 -8.636) (width 0.508) (layer F.Cu) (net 14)))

